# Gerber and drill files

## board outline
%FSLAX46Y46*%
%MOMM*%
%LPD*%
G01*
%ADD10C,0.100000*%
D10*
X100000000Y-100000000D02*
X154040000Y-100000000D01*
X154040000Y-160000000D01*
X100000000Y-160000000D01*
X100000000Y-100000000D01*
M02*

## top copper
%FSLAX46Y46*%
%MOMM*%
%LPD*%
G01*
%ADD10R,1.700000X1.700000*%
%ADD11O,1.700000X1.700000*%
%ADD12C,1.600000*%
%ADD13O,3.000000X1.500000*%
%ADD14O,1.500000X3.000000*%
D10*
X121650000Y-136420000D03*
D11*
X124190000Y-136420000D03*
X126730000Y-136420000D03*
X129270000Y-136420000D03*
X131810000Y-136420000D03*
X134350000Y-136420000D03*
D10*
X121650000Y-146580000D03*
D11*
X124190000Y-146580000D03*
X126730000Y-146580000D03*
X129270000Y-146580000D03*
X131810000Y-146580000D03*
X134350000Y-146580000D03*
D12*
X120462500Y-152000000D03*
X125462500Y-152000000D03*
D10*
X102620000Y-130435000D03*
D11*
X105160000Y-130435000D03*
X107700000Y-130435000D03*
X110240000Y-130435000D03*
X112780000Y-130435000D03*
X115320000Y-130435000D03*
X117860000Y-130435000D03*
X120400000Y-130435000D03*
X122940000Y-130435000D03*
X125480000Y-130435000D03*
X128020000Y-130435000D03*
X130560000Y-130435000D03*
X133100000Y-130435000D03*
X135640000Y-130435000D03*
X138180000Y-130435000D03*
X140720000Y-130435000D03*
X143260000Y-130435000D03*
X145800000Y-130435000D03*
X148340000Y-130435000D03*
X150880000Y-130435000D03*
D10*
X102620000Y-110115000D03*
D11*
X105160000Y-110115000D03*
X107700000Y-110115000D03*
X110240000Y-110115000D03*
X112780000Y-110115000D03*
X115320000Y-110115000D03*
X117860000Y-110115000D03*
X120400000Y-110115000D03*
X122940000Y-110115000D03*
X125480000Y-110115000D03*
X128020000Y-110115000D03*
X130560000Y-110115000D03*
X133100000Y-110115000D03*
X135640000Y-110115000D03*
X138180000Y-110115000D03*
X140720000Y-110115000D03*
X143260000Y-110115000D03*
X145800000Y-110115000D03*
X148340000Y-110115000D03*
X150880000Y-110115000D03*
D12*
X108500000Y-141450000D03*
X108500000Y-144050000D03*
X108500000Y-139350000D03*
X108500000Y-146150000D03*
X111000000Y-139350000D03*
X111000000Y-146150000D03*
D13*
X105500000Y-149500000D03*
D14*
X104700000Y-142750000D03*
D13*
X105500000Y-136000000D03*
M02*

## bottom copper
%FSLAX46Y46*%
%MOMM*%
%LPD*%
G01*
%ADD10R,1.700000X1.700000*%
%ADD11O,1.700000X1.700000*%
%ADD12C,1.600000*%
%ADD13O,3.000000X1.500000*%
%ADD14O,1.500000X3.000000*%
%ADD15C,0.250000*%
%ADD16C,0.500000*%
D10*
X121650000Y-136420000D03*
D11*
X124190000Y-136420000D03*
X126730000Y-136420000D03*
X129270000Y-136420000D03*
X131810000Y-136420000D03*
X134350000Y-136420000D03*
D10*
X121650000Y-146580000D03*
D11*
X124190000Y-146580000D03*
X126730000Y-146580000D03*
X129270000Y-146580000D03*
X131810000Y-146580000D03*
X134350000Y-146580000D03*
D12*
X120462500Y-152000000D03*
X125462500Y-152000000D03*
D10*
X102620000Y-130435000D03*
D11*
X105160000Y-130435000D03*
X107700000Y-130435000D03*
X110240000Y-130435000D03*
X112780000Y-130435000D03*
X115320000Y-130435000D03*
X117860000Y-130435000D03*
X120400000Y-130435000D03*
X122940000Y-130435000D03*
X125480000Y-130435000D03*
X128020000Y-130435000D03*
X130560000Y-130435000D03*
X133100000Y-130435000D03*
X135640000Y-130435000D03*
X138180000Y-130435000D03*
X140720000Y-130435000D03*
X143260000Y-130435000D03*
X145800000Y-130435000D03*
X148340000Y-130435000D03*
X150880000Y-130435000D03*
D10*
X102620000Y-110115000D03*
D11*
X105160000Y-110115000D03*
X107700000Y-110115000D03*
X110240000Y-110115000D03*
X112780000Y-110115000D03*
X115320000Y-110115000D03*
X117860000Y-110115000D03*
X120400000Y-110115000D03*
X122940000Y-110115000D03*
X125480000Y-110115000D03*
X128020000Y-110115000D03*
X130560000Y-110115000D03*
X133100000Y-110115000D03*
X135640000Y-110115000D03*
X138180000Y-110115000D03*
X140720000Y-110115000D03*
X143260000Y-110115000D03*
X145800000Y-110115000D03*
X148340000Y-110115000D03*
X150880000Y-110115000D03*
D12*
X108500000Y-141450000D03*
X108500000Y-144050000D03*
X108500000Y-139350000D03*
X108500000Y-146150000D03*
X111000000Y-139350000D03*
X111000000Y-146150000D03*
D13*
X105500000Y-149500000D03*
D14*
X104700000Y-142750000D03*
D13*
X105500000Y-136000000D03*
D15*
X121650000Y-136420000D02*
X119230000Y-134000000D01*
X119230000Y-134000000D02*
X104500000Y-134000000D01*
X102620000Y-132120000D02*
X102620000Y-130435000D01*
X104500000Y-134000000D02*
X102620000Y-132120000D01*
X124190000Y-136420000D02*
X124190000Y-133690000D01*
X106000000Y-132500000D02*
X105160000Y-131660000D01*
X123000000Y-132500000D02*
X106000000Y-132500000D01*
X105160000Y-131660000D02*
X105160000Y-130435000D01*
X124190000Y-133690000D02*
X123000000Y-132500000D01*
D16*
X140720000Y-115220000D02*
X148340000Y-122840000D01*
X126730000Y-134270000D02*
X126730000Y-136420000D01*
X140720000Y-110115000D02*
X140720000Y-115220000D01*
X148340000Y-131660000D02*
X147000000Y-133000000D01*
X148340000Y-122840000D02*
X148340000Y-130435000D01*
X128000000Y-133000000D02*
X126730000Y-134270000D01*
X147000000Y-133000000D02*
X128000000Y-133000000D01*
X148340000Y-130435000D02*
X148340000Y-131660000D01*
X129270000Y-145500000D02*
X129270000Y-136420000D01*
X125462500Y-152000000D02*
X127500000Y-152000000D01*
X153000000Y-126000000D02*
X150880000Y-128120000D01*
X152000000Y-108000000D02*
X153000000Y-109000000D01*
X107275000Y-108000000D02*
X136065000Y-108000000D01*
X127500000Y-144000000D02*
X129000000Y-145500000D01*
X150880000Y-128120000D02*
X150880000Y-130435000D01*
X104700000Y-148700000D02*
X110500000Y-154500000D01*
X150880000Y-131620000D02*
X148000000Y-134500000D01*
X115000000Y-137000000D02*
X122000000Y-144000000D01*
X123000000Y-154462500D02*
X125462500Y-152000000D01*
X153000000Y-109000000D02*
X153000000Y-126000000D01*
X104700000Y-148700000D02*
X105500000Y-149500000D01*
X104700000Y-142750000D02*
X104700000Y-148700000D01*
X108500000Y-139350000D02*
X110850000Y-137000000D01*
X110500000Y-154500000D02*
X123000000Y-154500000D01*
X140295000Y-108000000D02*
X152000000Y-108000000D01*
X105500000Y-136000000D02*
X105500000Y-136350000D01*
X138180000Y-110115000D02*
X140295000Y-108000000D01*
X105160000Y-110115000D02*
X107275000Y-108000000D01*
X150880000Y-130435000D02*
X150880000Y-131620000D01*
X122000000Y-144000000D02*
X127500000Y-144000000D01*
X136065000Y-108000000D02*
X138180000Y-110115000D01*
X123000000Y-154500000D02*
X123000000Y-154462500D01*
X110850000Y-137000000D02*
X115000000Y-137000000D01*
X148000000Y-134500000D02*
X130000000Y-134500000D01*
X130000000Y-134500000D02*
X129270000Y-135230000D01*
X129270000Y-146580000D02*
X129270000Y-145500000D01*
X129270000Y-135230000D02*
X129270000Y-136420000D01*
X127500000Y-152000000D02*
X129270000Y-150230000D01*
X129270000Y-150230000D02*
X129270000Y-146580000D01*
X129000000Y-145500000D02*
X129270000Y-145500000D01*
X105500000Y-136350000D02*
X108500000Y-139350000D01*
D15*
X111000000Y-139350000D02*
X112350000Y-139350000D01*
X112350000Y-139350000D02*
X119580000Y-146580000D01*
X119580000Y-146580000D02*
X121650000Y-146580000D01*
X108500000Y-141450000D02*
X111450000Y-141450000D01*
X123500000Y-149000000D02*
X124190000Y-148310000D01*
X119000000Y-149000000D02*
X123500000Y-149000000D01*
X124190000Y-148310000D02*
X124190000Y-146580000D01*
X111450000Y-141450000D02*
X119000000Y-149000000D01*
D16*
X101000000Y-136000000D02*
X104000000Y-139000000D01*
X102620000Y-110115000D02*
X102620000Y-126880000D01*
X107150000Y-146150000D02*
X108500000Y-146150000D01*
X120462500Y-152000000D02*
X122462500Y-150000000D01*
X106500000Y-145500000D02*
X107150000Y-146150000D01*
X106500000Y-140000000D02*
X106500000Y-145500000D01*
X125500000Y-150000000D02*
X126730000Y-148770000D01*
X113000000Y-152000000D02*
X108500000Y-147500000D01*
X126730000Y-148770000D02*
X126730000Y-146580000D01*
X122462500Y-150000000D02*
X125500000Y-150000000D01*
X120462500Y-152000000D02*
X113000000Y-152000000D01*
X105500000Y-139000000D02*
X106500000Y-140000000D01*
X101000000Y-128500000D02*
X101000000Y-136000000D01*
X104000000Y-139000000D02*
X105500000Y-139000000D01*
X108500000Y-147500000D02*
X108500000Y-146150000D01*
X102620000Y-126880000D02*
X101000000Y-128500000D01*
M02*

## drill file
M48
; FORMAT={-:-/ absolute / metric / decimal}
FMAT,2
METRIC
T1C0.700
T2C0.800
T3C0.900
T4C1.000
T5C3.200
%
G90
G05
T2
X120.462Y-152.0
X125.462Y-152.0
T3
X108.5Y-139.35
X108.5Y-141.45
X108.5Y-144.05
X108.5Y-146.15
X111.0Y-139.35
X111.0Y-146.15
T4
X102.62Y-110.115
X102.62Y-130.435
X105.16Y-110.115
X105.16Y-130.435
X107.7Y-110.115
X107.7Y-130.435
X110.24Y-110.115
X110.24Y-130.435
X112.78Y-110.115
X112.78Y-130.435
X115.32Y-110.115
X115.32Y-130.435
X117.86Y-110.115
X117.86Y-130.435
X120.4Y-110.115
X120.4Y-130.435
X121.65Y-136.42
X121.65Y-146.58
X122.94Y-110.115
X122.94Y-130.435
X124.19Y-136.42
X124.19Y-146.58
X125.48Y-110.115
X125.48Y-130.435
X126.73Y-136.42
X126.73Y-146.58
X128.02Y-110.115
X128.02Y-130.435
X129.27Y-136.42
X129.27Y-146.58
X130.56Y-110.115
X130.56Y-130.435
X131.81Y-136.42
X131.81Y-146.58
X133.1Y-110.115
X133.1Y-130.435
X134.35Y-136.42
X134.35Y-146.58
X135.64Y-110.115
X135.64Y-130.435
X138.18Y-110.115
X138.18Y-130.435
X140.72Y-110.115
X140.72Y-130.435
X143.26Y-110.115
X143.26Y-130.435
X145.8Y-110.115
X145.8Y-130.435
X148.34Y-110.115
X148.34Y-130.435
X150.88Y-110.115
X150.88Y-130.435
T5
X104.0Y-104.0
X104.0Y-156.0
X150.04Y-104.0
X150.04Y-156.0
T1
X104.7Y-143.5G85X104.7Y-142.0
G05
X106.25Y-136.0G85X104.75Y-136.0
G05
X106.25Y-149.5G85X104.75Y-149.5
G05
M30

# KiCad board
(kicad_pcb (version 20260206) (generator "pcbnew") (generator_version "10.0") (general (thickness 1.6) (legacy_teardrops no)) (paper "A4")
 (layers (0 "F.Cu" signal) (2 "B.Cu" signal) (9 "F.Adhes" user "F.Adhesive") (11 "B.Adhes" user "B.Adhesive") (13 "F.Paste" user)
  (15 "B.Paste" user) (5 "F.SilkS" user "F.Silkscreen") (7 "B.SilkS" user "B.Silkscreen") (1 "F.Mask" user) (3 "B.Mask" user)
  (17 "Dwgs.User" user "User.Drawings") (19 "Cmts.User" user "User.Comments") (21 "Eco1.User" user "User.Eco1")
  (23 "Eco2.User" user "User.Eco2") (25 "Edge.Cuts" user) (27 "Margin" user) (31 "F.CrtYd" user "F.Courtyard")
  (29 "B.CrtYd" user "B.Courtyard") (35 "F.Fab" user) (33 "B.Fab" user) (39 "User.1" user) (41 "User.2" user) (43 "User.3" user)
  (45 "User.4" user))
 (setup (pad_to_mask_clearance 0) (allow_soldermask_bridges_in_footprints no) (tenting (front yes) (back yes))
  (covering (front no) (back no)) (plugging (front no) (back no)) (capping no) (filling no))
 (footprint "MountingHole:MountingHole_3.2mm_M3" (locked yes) (layer "F.Cu") (at 150.04 104)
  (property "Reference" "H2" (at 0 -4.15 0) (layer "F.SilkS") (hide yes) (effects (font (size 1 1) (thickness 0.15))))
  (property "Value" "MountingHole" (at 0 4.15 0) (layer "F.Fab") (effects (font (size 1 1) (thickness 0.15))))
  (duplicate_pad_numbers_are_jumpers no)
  (pad "" np_thru_hole circle (at 0 0) (size 3.2 3.2) (drill 3.2) (layers "*.Cu" "*.Mask")))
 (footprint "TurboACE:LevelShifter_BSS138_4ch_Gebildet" (layer "F.Cu") (at 121.65 136.42 180)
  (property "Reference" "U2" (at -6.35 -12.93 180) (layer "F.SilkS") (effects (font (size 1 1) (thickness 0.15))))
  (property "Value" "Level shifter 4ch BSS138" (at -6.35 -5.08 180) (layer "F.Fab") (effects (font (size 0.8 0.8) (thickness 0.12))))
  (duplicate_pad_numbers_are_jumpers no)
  (pad "1" thru_hole rect (at 0 0 180) (size 1.7 1.7) (drill 1) (layers "*.Cu" "*.Mask") (remove_unused_layers no) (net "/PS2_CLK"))
  (pad "2" thru_hole oval (at -2.54 0 180) (size 1.7 1.7) (drill 1) (layers "*.Cu" "*.Mask") (remove_unused_layers no) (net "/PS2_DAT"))
  (pad "3" thru_hole oval (at -5.08 0 180) (size 1.7 1.7) (drill 1) (layers "*.Cu" "*.Mask") (remove_unused_layers no) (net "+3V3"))
  (pad "4" thru_hole oval (at -7.62 0 180) (size 1.7 1.7) (drill 1) (layers "*.Cu" "*.Mask") (remove_unused_layers no) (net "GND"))
  (pad "5" thru_hole oval (at -10.16 0 180) (size 1.7 1.7) (drill 1) (layers "*.Cu" "*.Mask") (remove_unused_layers no)
   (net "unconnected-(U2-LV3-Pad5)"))
  (pad "6" thru_hole oval (at -12.7 0 180) (size 1.7 1.7) (drill 1) (layers "*.Cu" "*.Mask") (remove_unused_layers no)
   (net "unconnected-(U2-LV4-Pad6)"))
  (pad "7" thru_hole rect (at 0 -10.16 180) (size 1.7 1.7) (drill 1) (layers "*.Cu" "*.Mask") (remove_unused_layers no) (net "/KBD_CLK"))
  (pad "8" thru_hole oval (at -2.54 -10.16 180) (size 1.7 1.7) (drill 1) (layers "*.Cu" "*.Mask") (remove_unused_layers no) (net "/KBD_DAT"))
  (pad "9" thru_hole oval (at -5.08 -10.16 180) (size 1.7 1.7) (drill 1) (layers "*.Cu" "*.Mask") (remove_unused_layers no) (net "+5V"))
  (pad "10" thru_hole oval (at -7.62 -10.16 180) (size 1.7 1.7) (drill 1) (layers "*.Cu" "*.Mask") (remove_unused_layers no) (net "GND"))
  (pad "11" thru_hole oval (at -10.16 -10.16 180) (size 1.7 1.7) (drill 1) (layers "*.Cu" "*.Mask") (remove_unused_layers no)
   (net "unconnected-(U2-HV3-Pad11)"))
  (pad "12" thru_hole oval (at -12.7 -10.16 180) (size 1.7 1.7) (drill 1) (layers "*.Cu" "*.Mask") (remove_unused_layers no)
   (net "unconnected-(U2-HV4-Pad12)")))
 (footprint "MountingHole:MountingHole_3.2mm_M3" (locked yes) (layer "F.Cu") (at 104 156)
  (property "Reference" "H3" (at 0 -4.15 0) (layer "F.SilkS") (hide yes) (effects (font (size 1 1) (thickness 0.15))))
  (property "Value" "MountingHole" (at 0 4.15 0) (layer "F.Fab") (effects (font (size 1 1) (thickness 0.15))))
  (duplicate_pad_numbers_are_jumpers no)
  (pad "" np_thru_hole circle (at 0 0) (size 3.2 3.2) (drill 3.2) (layers "*.Cu" "*.Mask")))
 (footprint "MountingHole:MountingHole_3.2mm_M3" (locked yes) (layer "F.Cu") (at 104 104)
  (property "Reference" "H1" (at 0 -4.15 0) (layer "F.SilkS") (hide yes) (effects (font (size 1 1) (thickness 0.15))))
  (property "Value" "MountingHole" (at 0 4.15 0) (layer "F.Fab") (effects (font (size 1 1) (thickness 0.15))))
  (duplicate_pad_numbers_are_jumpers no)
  (pad "" np_thru_hole circle (at 0 0) (size 3.2 3.2) (drill 3.2) (layers "*.Cu" "*.Mask")))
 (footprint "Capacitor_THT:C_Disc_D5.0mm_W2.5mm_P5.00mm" (layer "F.Cu") (at 120.4625 152)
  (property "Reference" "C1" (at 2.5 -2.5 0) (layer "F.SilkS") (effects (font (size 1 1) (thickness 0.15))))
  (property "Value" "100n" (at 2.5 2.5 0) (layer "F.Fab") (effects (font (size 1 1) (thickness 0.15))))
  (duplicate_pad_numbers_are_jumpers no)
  (pad "1" thru_hole circle (at 0 0) (size 1.6 1.6) (drill 0.8) (layers "*.Cu" "*.Mask") (remove_unused_layers no) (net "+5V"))
  (pad "2" thru_hole circle (at 5 0) (size 1.6 1.6) (drill 0.8) (layers "*.Cu" "*.Mask") (remove_unused_layers no) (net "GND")))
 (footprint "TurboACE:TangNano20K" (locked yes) (layer "F.Cu") (at 102.62 130.435)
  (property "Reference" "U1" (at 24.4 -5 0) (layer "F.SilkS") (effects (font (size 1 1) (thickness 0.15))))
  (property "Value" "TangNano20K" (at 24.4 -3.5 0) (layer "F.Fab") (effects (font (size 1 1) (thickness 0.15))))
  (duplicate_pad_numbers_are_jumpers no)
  (pad "1" thru_hole rect (at 0 0) (size 1.7 1.7) (drill 1) (layers "*.Cu" "*.Mask") (remove_unused_layers no) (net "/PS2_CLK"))
  (pad "2" thru_hole oval (at 2.54 0) (size 1.7 1.7) (drill 1) (layers "*.Cu" "*.Mask") (remove_unused_layers no) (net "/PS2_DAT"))
  (pad "3" thru_hole oval (at 5.08 0) (size 1.7 1.7) (drill 1) (layers "*.Cu" "*.Mask") (remove_unused_layers no)
   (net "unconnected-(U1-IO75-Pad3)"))
  (pad "4" thru_hole oval (at 7.62 0) (size 1.7 1.7) (drill 1) (layers "*.Cu" "*.Mask") (remove_unused_layers no)
   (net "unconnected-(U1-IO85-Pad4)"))
  (pad "5" thru_hole oval (at 10.16 0) (size 1.7 1.7) (drill 1) (layers "*.Cu" "*.Mask") (remove_unused_layers no)
   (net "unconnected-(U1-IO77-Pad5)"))
  (pad "6" thru_hole oval (at 12.7 0) (size 1.7 1.7) (drill 1) (layers "*.Cu" "*.Mask") (remove_unused_layers no)
   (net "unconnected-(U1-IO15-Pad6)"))
  (pad "7" thru_hole oval (at 15.24 0) (size 1.7 1.7) (drill 1) (layers "*.Cu" "*.Mask") (remove_unused_layers no)
   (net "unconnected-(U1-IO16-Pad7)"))
  (pad "8" thru_hole oval (at 17.78 0) (size 1.7 1.7) (drill 1) (layers "*.Cu" "*.Mask") (remove_unused_layers no)
   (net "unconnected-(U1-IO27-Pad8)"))
  (pad "9" thru_hole oval (at 20.32 0) (size 1.7 1.7) (drill 1) (layers "*.Cu" "*.Mask") (remove_unused_layers no)
   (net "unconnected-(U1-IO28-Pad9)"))
  (pad "10" thru_hole oval (at 22.86 0) (size 1.7 1.7) (drill 1) (layers "*.Cu" "*.Mask") (remove_unused_layers no)
   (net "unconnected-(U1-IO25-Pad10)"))
  (pad "11" thru_hole oval (at 25.4 0) (size 1.7 1.7) (drill 1) (layers "*.Cu" "*.Mask") (remove_unused_layers no)
   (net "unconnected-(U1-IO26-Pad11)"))
  (pad "12" thru_hole oval (at 27.94 0) (size 1.7 1.7) (drill 1) (layers "*.Cu" "*.Mask") (remove_unused_layers no)
   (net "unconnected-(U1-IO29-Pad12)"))
  (pad "13" thru_hole oval (at 30.48 0) (size 1.7 1.7) (drill 1) (layers "*.Cu" "*.Mask") (remove_unused_layers no)
   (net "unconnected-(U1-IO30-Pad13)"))
  (pad "14" thru_hole oval (at 33.02 0) (size 1.7 1.7) (drill 1) (layers "*.Cu" "*.Mask") (remove_unused_layers no)
   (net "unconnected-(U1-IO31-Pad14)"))
  (pad "15" thru_hole oval (at 35.56 0) (size 1.7 1.7) (drill 1) (layers "*.Cu" "*.Mask") (remove_unused_layers no)
   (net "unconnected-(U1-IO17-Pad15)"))
  (pad "16" thru_hole oval (at 38.1 0) (size 1.7 1.7) (drill 1) (layers "*.Cu" "*.Mask") (remove_unused_layers no)
   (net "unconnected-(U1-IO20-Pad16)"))
  (pad "17" thru_hole oval (at 40.64 0) (size 1.7 1.7) (drill 1) (layers "*.Cu" "*.Mask") (remove_unused_layers no)
   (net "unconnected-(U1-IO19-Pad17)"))
  (pad "18" thru_hole oval (at 43.18 0) (size 1.7 1.7) (drill 1) (layers "*.Cu" "*.Mask") (remove_unused_layers no)
   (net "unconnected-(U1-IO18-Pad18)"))
  (pad "19" thru_hole oval (at 45.72 0) (size 1.7 1.7) (drill 1) (layers "*.Cu" "*.Mask") (remove_unused_layers no) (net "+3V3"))
  (pad "20" thru_hole oval (at 48.26 0) (size 1.7 1.7) (drill 1) (layers "*.Cu" "*.Mask") (remove_unused_layers no) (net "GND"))
  (pad "21" thru_hole rect (at 0 -20.32) (size 1.7 1.7) (drill 1) (layers "*.Cu" "*.Mask") (remove_unused_layers no) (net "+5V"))
  (pad "22" thru_hole oval (at 2.54 -20.32) (size 1.7 1.7) (drill 1) (layers "*.Cu" "*.Mask") (remove_unused_layers no) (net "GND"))
  (pad "23" thru_hole oval (at 5.08 -20.32) (size 1.7 1.7) (drill 1) (layers "*.Cu" "*.Mask") (remove_unused_layers no)
   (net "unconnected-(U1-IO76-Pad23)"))
  (pad "24" thru_hole oval (at 7.62 -20.32) (size 1.7 1.7) (drill 1) (layers "*.Cu" "*.Mask") (remove_unused_layers no)
   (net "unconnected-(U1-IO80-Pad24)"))
  (pad "25" thru_hole oval (at 10.16 -20.32) (size 1.7 1.7) (drill 1) (layers "*.Cu" "*.Mask") (remove_unused_layers no)
   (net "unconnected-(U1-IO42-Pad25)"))
  (pad "26" thru_hole oval (at 12.7 -20.32) (size 1.7 1.7) (drill 1) (layers "*.Cu" "*.Mask") (remove_unused_layers no)
   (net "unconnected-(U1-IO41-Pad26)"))
  (pad "27" thru_hole oval (at 15.24 -20.32) (size 1.7 1.7) (drill 1) (layers "*.Cu" "*.Mask") (remove_unused_layers no)
   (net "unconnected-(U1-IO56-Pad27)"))
  (pad "28" thru_hole oval (at 17.78 -20.32) (size 1.7 1.7) (drill 1) (layers "*.Cu" "*.Mask") (remove_unused_layers no)
   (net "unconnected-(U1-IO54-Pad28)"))
  (pad "29" thru_hole oval (at 20.32 -20.32) (size 1.7 1.7) (drill 1) (layers "*.Cu" "*.Mask") (remove_unused_layers no)
   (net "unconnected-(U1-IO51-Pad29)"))
  (pad "30" thru_hole oval (at 22.86 -20.32) (size 1.7 1.7) (drill 1) (layers "*.Cu" "*.Mask") (remove_unused_layers no)
   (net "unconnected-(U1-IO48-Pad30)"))
  (pad "31" thru_hole oval (at 25.4 -20.32) (size 1.7 1.7) (drill 1) (layers "*.Cu" "*.Mask") (remove_unused_layers no)
   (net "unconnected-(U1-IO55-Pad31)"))
  (pad "32" thru_hole oval (at 27.94 -20.32) (size 1.7 1.7) (drill 1) (layers "*.Cu" "*.Mask") (remove_unused_layers no)
   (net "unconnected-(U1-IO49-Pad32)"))
  (pad "33" thru_hole oval (at 30.48 -20.32) (size 1.7 1.7) (drill 1) (layers "*.Cu" "*.Mask") (remove_unused_layers no)
   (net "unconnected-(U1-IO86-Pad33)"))
  (pad "34" thru_hole oval (at 33.02 -20.32) (size 1.7 1.7) (drill 1) (layers "*.Cu" "*.Mask") (remove_unused_layers no)
   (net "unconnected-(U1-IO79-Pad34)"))
  (pad "35" thru_hole oval (at 35.56 -20.32) (size 1.7 1.7) (drill 1) (layers "*.Cu" "*.Mask") (remove_unused_layers no) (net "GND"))
  (pad "36" thru_hole oval (at 38.1 -20.32) (size 1.7 1.7) (drill 1) (layers "*.Cu" "*.Mask") (remove_unused_layers no) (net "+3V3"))
  (pad "37" thru_hole oval (at 40.64 -20.32) (size 1.7 1.7) (drill 1) (layers "*.Cu" "*.Mask") (remove_unused_layers no)
   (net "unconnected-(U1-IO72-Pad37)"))
  (pad "38" thru_hole oval (at 43.18 -20.32) (size 1.7 1.7) (drill 1) (layers "*.Cu" "*.Mask") (remove_unused_layers no)
   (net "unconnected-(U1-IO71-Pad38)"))
  (pad "39" thru_hole oval (at 45.72 -20.32) (size 1.7 1.7) (drill 1) (layers "*.Cu" "*.Mask") (remove_unused_layers no)
   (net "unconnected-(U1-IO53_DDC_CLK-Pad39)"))
  (pad "40" thru_hole oval (at 48.26 -20.32) (size 1.7 1.7) (drill 1) (layers "*.Cu" "*.Mask") (remove_unused_layers no)
   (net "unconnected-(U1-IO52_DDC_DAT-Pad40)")))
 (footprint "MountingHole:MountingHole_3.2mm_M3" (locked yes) (layer "F.Cu") (at 150.04 156)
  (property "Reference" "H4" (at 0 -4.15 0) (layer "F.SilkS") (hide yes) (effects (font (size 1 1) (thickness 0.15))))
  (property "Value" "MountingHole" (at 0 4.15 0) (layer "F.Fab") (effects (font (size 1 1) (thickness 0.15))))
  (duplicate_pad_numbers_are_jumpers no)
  (pad "" np_thru_hole circle (at 0 0) (size 3.2 3.2) (drill 3.2) (layers "*.Cu" "*.Mask")))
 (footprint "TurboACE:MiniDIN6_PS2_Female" (layer "F.Cu") (at 100 142.75 90)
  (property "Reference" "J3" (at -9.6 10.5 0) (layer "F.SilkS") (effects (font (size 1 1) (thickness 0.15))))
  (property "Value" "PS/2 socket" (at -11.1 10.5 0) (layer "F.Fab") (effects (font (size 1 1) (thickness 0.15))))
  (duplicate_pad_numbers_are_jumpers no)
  (pad "1" thru_hole circle (at 1.3 8.5 90) (size 1.6 1.6) (drill 0.9) (layers "*.Cu" "*.Mask") (remove_unused_layers no) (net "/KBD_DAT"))
  (pad "2" thru_hole circle (at -1.3 8.5 90) (size 1.6 1.6) (drill 0.9) (layers "*.Cu" "*.Mask") (remove_unused_layers no)
   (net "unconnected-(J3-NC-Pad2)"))
  (pad "3" thru_hole circle (at 3.4 8.5 90) (size 1.6 1.6) (drill 0.9) (layers "*.Cu" "*.Mask") (remove_unused_layers no) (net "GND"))
  (pad "4" thru_hole circle (at -3.4 8.5 90) (size 1.6 1.6) (drill 0.9) (layers "*.Cu" "*.Mask") (remove_unused_layers no) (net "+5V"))
  (pad "5" thru_hole circle (at 3.4 11 90) (size 1.6 1.6) (drill 0.9) (layers "*.Cu" "*.Mask") (remove_unused_layers no) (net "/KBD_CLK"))
  (pad "6" thru_hole circle (at -3.4 11 90) (size 1.6 1.6) (drill 0.9) (layers "*.Cu" "*.Mask") (remove_unused_layers no)
   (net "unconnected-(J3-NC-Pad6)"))
  (pad "SH" thru_hole oval (at -6.75 5.5 180) (size 3 1.5) (drill oval 2.2 0.7) (layers "*.Cu" "*.Mask") (remove_unused_layers no)
   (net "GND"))
  (pad "SH" thru_hole oval (at 0 4.7 90) (size 3 1.5) (drill oval 2.2 0.7) (layers "*.Cu" "*.Mask") (remove_unused_layers no) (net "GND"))
  (pad "SH" thru_hole oval (at 6.75 5.5 180) (size 3 1.5) (drill oval 2.2 0.7) (layers "*.Cu" "*.Mask") (remove_unused_layers no)
   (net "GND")))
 (gr_rect (start 100 100) (end 154.04 160) (stroke (width 0.1) (type default)) (fill no) (layer "Edge.Cuts"))
 (segment (start 121.65 136.42) (end 119.23 134) (width 0.25) (layer "B.Cu") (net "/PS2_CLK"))
 (segment (start 119.23 134) (end 104.5 134) (width 0.25) (layer "B.Cu") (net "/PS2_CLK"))
 (segment (start 102.62 132.12) (end 102.62 130.435) (width 0.25) (layer "B.Cu") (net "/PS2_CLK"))
 (segment (start 104.5 134) (end 102.62 132.12) (width 0.25) (layer "B.Cu") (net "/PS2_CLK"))
 (segment (start 124.19 136.42) (end 124.19 133.69) (width 0.25) (layer "B.Cu") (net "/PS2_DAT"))
 (segment (start 106 132.5) (end 105.16 131.66) (width 0.25) (layer "B.Cu") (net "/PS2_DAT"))
 (segment (start 123 132.5) (end 106 132.5) (width 0.25) (layer "B.Cu") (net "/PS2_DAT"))
 (segment (start 105.16 131.66) (end 105.16 130.435) (width 0.25) (layer "B.Cu") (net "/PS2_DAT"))
 (segment (start 124.19 133.69) (end 123 132.5) (width 0.25) (layer "B.Cu") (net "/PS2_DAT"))
 (segment (start 140.72 115.22) (end 148.34 122.84) (width 0.5) (layer "B.Cu") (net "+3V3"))
 (segment (start 126.73 134.27) (end 126.73 136.42) (width 0.5) (layer "B.Cu") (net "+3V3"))
 (segment (start 140.72 110.115) (end 140.72 115.22) (width 0.5) (layer "B.Cu") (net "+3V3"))
 (segment (start 148.34 131.66) (end 147 133) (width 0.5) (layer "B.Cu") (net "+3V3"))
 (segment (start 148.34 122.84) (end 148.34 130.435) (width 0.5) (layer "B.Cu") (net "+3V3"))
 (segment (start 128 133) (end 126.73 134.27) (width 0.5) (layer "B.Cu") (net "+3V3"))
 (segment (start 147 133) (end 128 133) (width 0.5) (layer "B.Cu") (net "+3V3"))
 (segment (start 148.34 130.435) (end 148.34 131.66) (width 0.5) (layer "B.Cu") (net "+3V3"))
 (segment (start 129.27 145.5) (end 129.27 136.42) (width 0.5) (layer "B.Cu") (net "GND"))
 (segment (start 125.4625 152) (end 127.5 152) (width 0.5) (layer "B.Cu") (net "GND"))
 (segment (start 153 126) (end 150.88 128.12) (width 0.5) (layer "B.Cu") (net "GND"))
 (segment (start 152 108) (end 153 109) (width 0.5) (layer "B.Cu") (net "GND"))
 (segment (start 107.275 108) (end 136.065 108) (width 0.5) (layer "B.Cu") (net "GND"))
 (segment (start 127.5 144) (end 129 145.5) (width 0.5) (layer "B.Cu") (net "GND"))
 (segment (start 150.88 128.12) (end 150.88 130.435) (width 0.5) (layer "B.Cu") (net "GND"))
 (segment (start 104.7 148.7) (end 110.5 154.5) (width 0.5) (layer "B.Cu") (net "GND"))
 (segment (start 150.88 131.62) (end 148 134.5) (width 0.5) (layer "B.Cu") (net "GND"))
 (segment (start 115 137) (end 122 144) (width 0.5) (layer "B.Cu") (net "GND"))
 (segment (start 123 154.4625) (end 125.4625 152) (width 0.5) (layer "B.Cu") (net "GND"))
 (segment (start 153 109) (end 153 126) (width 0.5) (layer "B.Cu") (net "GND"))
 (segment (start 104.7 148.7) (end 105.5 149.5) (width 0.5) (layer "B.Cu") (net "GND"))
 (segment (start 104.7 142.75) (end 104.7 148.7) (width 0.5) (layer "B.Cu") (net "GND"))
 (segment (start 108.5 139.35) (end 110.85 137) (width 0.5) (layer "B.Cu") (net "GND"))
 (segment (start 110.5 154.5) (end 123 154.5) (width 0.5) (layer "B.Cu") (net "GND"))
 (segment (start 140.295 108) (end 152 108) (width 0.5) (layer "B.Cu") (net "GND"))
 (segment (start 105.5 136) (end 105.5 136.35) (width 0.5) (layer "B.Cu") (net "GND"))
 (segment (start 138.18 110.115) (end 140.295 108) (width 0.5) (layer "B.Cu") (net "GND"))
 (segment (start 105.16 110.115) (end 107.275 108) (width 0.5) (layer "B.Cu") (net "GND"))
 (segment (start 150.88 130.435) (end 150.88 131.62) (width 0.5) (layer "B.Cu") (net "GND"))
 (segment (start 122 144) (end 127.5 144) (width 0.5) (layer "B.Cu") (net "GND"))
 (segment (start 136.065 108) (end 138.18 110.115) (width 0.5) (layer "B.Cu") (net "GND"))
 (segment (start 123 154.5) (end 123 154.4625) (width 0.5) (layer "B.Cu") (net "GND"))
 (segment (start 110.85 137) (end 115 137) (width 0.5) (layer "B.Cu") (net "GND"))
 (segment (start 148 134.5) (end 130 134.5) (width 0.5) (layer "B.Cu") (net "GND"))
 (segment (start 130 134.5) (end 129.27 135.23) (width 0.5) (layer "B.Cu") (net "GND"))
 (segment (start 129.27 146.58) (end 129.27 145.5) (width 0.5) (layer "B.Cu") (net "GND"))
 (segment (start 129.27 135.23) (end 129.27 136.42) (width 0.5) (layer "B.Cu") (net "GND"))
 (segment (start 127.5 152) (end 129.27 150.23) (width 0.5) (layer "B.Cu") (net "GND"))
 (segment (start 129.27 150.23) (end 129.27 146.58) (width 0.5) (layer "B.Cu") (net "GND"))
 (segment (start 129 145.5) (end 129.27 145.5) (width 0.5) (layer "B.Cu") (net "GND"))
 (segment (start 105.5 136.35) (end 108.5 139.35) (width 0.5) (layer "B.Cu") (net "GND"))
 (segment (start 111 139.35) (end 112.35 139.35) (width 0.25) (layer "B.Cu") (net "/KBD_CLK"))
 (segment (start 112.35 139.35) (end 119.58 146.58) (width 0.25) (layer "B.Cu") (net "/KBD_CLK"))
 (segment (start 119.58 146.58) (end 121.65 146.58) (width 0.25) (layer "B.Cu") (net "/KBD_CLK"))
 (segment (start 108.5 141.45) (end 111.45 141.45) (width 0.25) (layer "B.Cu") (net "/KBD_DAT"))
 (segment (start 123.5 149) (end 124.19 148.31) (width 0.25) (layer "B.Cu") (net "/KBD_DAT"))
 (segment (start 119 149) (end 123.5 149) (width 0.25) (layer "B.Cu") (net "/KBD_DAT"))
 (segment (start 124.19 148.31) (end 124.19 146.58) (width 0.25) (layer "B.Cu") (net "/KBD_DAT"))
 (segment (start 111.45 141.45) (end 119 149) (width 0.25) (layer "B.Cu") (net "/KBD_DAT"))
 (segment (start 101 136) (end 104 139) (width 0.5) (layer "B.Cu") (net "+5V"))
 (segment (start 102.62 110.115) (end 102.62 126.88) (width 0.5) (layer "B.Cu") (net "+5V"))
 (segment (start 107.15 146.15) (end 108.5 146.15) (width 0.5) (layer "B.Cu") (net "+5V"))
 (segment (start 120.4625 152) (end 122.4625 150) (width 0.5) (layer "B.Cu") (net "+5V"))
 (segment (start 106.5 145.5) (end 107.15 146.15) (width 0.5) (layer "B.Cu") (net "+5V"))
 (segment (start 106.5 140) (end 106.5 145.5) (width 0.5) (layer "B.Cu") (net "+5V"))
 (segment (start 125.5 150) (end 126.73 148.77) (width 0.5) (layer "B.Cu") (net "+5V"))
 (segment (start 113 152) (end 108.5 147.5) (width 0.5) (layer "B.Cu") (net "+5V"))
 (segment (start 126.73 148.77) (end 126.73 146.58) (width 0.5) (layer "B.Cu") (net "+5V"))
 (segment (start 122.4625 150) (end 125.5 150) (width 0.5) (layer "B.Cu") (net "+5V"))
 (segment (start 120.4625 152) (end 113 152) (width 0.5) (layer "B.Cu") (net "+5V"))
 (segment (start 105.5 139) (end 106.5 140) (width 0.5) (layer "B.Cu") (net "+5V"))
 (segment (start 101 128.5) (end 101 136) (width 0.5) (layer "B.Cu") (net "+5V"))
 (segment (start 104 139) (end 105.5 139) (width 0.5) (layer "B.Cu") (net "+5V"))
 (segment (start 108.5 147.5) (end 108.5 146.15) (width 0.5) (layer "B.Cu") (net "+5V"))
 (segment (start 102.62 126.88) (end 101 128.5) (width 0.5) (layer "B.Cu") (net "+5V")))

